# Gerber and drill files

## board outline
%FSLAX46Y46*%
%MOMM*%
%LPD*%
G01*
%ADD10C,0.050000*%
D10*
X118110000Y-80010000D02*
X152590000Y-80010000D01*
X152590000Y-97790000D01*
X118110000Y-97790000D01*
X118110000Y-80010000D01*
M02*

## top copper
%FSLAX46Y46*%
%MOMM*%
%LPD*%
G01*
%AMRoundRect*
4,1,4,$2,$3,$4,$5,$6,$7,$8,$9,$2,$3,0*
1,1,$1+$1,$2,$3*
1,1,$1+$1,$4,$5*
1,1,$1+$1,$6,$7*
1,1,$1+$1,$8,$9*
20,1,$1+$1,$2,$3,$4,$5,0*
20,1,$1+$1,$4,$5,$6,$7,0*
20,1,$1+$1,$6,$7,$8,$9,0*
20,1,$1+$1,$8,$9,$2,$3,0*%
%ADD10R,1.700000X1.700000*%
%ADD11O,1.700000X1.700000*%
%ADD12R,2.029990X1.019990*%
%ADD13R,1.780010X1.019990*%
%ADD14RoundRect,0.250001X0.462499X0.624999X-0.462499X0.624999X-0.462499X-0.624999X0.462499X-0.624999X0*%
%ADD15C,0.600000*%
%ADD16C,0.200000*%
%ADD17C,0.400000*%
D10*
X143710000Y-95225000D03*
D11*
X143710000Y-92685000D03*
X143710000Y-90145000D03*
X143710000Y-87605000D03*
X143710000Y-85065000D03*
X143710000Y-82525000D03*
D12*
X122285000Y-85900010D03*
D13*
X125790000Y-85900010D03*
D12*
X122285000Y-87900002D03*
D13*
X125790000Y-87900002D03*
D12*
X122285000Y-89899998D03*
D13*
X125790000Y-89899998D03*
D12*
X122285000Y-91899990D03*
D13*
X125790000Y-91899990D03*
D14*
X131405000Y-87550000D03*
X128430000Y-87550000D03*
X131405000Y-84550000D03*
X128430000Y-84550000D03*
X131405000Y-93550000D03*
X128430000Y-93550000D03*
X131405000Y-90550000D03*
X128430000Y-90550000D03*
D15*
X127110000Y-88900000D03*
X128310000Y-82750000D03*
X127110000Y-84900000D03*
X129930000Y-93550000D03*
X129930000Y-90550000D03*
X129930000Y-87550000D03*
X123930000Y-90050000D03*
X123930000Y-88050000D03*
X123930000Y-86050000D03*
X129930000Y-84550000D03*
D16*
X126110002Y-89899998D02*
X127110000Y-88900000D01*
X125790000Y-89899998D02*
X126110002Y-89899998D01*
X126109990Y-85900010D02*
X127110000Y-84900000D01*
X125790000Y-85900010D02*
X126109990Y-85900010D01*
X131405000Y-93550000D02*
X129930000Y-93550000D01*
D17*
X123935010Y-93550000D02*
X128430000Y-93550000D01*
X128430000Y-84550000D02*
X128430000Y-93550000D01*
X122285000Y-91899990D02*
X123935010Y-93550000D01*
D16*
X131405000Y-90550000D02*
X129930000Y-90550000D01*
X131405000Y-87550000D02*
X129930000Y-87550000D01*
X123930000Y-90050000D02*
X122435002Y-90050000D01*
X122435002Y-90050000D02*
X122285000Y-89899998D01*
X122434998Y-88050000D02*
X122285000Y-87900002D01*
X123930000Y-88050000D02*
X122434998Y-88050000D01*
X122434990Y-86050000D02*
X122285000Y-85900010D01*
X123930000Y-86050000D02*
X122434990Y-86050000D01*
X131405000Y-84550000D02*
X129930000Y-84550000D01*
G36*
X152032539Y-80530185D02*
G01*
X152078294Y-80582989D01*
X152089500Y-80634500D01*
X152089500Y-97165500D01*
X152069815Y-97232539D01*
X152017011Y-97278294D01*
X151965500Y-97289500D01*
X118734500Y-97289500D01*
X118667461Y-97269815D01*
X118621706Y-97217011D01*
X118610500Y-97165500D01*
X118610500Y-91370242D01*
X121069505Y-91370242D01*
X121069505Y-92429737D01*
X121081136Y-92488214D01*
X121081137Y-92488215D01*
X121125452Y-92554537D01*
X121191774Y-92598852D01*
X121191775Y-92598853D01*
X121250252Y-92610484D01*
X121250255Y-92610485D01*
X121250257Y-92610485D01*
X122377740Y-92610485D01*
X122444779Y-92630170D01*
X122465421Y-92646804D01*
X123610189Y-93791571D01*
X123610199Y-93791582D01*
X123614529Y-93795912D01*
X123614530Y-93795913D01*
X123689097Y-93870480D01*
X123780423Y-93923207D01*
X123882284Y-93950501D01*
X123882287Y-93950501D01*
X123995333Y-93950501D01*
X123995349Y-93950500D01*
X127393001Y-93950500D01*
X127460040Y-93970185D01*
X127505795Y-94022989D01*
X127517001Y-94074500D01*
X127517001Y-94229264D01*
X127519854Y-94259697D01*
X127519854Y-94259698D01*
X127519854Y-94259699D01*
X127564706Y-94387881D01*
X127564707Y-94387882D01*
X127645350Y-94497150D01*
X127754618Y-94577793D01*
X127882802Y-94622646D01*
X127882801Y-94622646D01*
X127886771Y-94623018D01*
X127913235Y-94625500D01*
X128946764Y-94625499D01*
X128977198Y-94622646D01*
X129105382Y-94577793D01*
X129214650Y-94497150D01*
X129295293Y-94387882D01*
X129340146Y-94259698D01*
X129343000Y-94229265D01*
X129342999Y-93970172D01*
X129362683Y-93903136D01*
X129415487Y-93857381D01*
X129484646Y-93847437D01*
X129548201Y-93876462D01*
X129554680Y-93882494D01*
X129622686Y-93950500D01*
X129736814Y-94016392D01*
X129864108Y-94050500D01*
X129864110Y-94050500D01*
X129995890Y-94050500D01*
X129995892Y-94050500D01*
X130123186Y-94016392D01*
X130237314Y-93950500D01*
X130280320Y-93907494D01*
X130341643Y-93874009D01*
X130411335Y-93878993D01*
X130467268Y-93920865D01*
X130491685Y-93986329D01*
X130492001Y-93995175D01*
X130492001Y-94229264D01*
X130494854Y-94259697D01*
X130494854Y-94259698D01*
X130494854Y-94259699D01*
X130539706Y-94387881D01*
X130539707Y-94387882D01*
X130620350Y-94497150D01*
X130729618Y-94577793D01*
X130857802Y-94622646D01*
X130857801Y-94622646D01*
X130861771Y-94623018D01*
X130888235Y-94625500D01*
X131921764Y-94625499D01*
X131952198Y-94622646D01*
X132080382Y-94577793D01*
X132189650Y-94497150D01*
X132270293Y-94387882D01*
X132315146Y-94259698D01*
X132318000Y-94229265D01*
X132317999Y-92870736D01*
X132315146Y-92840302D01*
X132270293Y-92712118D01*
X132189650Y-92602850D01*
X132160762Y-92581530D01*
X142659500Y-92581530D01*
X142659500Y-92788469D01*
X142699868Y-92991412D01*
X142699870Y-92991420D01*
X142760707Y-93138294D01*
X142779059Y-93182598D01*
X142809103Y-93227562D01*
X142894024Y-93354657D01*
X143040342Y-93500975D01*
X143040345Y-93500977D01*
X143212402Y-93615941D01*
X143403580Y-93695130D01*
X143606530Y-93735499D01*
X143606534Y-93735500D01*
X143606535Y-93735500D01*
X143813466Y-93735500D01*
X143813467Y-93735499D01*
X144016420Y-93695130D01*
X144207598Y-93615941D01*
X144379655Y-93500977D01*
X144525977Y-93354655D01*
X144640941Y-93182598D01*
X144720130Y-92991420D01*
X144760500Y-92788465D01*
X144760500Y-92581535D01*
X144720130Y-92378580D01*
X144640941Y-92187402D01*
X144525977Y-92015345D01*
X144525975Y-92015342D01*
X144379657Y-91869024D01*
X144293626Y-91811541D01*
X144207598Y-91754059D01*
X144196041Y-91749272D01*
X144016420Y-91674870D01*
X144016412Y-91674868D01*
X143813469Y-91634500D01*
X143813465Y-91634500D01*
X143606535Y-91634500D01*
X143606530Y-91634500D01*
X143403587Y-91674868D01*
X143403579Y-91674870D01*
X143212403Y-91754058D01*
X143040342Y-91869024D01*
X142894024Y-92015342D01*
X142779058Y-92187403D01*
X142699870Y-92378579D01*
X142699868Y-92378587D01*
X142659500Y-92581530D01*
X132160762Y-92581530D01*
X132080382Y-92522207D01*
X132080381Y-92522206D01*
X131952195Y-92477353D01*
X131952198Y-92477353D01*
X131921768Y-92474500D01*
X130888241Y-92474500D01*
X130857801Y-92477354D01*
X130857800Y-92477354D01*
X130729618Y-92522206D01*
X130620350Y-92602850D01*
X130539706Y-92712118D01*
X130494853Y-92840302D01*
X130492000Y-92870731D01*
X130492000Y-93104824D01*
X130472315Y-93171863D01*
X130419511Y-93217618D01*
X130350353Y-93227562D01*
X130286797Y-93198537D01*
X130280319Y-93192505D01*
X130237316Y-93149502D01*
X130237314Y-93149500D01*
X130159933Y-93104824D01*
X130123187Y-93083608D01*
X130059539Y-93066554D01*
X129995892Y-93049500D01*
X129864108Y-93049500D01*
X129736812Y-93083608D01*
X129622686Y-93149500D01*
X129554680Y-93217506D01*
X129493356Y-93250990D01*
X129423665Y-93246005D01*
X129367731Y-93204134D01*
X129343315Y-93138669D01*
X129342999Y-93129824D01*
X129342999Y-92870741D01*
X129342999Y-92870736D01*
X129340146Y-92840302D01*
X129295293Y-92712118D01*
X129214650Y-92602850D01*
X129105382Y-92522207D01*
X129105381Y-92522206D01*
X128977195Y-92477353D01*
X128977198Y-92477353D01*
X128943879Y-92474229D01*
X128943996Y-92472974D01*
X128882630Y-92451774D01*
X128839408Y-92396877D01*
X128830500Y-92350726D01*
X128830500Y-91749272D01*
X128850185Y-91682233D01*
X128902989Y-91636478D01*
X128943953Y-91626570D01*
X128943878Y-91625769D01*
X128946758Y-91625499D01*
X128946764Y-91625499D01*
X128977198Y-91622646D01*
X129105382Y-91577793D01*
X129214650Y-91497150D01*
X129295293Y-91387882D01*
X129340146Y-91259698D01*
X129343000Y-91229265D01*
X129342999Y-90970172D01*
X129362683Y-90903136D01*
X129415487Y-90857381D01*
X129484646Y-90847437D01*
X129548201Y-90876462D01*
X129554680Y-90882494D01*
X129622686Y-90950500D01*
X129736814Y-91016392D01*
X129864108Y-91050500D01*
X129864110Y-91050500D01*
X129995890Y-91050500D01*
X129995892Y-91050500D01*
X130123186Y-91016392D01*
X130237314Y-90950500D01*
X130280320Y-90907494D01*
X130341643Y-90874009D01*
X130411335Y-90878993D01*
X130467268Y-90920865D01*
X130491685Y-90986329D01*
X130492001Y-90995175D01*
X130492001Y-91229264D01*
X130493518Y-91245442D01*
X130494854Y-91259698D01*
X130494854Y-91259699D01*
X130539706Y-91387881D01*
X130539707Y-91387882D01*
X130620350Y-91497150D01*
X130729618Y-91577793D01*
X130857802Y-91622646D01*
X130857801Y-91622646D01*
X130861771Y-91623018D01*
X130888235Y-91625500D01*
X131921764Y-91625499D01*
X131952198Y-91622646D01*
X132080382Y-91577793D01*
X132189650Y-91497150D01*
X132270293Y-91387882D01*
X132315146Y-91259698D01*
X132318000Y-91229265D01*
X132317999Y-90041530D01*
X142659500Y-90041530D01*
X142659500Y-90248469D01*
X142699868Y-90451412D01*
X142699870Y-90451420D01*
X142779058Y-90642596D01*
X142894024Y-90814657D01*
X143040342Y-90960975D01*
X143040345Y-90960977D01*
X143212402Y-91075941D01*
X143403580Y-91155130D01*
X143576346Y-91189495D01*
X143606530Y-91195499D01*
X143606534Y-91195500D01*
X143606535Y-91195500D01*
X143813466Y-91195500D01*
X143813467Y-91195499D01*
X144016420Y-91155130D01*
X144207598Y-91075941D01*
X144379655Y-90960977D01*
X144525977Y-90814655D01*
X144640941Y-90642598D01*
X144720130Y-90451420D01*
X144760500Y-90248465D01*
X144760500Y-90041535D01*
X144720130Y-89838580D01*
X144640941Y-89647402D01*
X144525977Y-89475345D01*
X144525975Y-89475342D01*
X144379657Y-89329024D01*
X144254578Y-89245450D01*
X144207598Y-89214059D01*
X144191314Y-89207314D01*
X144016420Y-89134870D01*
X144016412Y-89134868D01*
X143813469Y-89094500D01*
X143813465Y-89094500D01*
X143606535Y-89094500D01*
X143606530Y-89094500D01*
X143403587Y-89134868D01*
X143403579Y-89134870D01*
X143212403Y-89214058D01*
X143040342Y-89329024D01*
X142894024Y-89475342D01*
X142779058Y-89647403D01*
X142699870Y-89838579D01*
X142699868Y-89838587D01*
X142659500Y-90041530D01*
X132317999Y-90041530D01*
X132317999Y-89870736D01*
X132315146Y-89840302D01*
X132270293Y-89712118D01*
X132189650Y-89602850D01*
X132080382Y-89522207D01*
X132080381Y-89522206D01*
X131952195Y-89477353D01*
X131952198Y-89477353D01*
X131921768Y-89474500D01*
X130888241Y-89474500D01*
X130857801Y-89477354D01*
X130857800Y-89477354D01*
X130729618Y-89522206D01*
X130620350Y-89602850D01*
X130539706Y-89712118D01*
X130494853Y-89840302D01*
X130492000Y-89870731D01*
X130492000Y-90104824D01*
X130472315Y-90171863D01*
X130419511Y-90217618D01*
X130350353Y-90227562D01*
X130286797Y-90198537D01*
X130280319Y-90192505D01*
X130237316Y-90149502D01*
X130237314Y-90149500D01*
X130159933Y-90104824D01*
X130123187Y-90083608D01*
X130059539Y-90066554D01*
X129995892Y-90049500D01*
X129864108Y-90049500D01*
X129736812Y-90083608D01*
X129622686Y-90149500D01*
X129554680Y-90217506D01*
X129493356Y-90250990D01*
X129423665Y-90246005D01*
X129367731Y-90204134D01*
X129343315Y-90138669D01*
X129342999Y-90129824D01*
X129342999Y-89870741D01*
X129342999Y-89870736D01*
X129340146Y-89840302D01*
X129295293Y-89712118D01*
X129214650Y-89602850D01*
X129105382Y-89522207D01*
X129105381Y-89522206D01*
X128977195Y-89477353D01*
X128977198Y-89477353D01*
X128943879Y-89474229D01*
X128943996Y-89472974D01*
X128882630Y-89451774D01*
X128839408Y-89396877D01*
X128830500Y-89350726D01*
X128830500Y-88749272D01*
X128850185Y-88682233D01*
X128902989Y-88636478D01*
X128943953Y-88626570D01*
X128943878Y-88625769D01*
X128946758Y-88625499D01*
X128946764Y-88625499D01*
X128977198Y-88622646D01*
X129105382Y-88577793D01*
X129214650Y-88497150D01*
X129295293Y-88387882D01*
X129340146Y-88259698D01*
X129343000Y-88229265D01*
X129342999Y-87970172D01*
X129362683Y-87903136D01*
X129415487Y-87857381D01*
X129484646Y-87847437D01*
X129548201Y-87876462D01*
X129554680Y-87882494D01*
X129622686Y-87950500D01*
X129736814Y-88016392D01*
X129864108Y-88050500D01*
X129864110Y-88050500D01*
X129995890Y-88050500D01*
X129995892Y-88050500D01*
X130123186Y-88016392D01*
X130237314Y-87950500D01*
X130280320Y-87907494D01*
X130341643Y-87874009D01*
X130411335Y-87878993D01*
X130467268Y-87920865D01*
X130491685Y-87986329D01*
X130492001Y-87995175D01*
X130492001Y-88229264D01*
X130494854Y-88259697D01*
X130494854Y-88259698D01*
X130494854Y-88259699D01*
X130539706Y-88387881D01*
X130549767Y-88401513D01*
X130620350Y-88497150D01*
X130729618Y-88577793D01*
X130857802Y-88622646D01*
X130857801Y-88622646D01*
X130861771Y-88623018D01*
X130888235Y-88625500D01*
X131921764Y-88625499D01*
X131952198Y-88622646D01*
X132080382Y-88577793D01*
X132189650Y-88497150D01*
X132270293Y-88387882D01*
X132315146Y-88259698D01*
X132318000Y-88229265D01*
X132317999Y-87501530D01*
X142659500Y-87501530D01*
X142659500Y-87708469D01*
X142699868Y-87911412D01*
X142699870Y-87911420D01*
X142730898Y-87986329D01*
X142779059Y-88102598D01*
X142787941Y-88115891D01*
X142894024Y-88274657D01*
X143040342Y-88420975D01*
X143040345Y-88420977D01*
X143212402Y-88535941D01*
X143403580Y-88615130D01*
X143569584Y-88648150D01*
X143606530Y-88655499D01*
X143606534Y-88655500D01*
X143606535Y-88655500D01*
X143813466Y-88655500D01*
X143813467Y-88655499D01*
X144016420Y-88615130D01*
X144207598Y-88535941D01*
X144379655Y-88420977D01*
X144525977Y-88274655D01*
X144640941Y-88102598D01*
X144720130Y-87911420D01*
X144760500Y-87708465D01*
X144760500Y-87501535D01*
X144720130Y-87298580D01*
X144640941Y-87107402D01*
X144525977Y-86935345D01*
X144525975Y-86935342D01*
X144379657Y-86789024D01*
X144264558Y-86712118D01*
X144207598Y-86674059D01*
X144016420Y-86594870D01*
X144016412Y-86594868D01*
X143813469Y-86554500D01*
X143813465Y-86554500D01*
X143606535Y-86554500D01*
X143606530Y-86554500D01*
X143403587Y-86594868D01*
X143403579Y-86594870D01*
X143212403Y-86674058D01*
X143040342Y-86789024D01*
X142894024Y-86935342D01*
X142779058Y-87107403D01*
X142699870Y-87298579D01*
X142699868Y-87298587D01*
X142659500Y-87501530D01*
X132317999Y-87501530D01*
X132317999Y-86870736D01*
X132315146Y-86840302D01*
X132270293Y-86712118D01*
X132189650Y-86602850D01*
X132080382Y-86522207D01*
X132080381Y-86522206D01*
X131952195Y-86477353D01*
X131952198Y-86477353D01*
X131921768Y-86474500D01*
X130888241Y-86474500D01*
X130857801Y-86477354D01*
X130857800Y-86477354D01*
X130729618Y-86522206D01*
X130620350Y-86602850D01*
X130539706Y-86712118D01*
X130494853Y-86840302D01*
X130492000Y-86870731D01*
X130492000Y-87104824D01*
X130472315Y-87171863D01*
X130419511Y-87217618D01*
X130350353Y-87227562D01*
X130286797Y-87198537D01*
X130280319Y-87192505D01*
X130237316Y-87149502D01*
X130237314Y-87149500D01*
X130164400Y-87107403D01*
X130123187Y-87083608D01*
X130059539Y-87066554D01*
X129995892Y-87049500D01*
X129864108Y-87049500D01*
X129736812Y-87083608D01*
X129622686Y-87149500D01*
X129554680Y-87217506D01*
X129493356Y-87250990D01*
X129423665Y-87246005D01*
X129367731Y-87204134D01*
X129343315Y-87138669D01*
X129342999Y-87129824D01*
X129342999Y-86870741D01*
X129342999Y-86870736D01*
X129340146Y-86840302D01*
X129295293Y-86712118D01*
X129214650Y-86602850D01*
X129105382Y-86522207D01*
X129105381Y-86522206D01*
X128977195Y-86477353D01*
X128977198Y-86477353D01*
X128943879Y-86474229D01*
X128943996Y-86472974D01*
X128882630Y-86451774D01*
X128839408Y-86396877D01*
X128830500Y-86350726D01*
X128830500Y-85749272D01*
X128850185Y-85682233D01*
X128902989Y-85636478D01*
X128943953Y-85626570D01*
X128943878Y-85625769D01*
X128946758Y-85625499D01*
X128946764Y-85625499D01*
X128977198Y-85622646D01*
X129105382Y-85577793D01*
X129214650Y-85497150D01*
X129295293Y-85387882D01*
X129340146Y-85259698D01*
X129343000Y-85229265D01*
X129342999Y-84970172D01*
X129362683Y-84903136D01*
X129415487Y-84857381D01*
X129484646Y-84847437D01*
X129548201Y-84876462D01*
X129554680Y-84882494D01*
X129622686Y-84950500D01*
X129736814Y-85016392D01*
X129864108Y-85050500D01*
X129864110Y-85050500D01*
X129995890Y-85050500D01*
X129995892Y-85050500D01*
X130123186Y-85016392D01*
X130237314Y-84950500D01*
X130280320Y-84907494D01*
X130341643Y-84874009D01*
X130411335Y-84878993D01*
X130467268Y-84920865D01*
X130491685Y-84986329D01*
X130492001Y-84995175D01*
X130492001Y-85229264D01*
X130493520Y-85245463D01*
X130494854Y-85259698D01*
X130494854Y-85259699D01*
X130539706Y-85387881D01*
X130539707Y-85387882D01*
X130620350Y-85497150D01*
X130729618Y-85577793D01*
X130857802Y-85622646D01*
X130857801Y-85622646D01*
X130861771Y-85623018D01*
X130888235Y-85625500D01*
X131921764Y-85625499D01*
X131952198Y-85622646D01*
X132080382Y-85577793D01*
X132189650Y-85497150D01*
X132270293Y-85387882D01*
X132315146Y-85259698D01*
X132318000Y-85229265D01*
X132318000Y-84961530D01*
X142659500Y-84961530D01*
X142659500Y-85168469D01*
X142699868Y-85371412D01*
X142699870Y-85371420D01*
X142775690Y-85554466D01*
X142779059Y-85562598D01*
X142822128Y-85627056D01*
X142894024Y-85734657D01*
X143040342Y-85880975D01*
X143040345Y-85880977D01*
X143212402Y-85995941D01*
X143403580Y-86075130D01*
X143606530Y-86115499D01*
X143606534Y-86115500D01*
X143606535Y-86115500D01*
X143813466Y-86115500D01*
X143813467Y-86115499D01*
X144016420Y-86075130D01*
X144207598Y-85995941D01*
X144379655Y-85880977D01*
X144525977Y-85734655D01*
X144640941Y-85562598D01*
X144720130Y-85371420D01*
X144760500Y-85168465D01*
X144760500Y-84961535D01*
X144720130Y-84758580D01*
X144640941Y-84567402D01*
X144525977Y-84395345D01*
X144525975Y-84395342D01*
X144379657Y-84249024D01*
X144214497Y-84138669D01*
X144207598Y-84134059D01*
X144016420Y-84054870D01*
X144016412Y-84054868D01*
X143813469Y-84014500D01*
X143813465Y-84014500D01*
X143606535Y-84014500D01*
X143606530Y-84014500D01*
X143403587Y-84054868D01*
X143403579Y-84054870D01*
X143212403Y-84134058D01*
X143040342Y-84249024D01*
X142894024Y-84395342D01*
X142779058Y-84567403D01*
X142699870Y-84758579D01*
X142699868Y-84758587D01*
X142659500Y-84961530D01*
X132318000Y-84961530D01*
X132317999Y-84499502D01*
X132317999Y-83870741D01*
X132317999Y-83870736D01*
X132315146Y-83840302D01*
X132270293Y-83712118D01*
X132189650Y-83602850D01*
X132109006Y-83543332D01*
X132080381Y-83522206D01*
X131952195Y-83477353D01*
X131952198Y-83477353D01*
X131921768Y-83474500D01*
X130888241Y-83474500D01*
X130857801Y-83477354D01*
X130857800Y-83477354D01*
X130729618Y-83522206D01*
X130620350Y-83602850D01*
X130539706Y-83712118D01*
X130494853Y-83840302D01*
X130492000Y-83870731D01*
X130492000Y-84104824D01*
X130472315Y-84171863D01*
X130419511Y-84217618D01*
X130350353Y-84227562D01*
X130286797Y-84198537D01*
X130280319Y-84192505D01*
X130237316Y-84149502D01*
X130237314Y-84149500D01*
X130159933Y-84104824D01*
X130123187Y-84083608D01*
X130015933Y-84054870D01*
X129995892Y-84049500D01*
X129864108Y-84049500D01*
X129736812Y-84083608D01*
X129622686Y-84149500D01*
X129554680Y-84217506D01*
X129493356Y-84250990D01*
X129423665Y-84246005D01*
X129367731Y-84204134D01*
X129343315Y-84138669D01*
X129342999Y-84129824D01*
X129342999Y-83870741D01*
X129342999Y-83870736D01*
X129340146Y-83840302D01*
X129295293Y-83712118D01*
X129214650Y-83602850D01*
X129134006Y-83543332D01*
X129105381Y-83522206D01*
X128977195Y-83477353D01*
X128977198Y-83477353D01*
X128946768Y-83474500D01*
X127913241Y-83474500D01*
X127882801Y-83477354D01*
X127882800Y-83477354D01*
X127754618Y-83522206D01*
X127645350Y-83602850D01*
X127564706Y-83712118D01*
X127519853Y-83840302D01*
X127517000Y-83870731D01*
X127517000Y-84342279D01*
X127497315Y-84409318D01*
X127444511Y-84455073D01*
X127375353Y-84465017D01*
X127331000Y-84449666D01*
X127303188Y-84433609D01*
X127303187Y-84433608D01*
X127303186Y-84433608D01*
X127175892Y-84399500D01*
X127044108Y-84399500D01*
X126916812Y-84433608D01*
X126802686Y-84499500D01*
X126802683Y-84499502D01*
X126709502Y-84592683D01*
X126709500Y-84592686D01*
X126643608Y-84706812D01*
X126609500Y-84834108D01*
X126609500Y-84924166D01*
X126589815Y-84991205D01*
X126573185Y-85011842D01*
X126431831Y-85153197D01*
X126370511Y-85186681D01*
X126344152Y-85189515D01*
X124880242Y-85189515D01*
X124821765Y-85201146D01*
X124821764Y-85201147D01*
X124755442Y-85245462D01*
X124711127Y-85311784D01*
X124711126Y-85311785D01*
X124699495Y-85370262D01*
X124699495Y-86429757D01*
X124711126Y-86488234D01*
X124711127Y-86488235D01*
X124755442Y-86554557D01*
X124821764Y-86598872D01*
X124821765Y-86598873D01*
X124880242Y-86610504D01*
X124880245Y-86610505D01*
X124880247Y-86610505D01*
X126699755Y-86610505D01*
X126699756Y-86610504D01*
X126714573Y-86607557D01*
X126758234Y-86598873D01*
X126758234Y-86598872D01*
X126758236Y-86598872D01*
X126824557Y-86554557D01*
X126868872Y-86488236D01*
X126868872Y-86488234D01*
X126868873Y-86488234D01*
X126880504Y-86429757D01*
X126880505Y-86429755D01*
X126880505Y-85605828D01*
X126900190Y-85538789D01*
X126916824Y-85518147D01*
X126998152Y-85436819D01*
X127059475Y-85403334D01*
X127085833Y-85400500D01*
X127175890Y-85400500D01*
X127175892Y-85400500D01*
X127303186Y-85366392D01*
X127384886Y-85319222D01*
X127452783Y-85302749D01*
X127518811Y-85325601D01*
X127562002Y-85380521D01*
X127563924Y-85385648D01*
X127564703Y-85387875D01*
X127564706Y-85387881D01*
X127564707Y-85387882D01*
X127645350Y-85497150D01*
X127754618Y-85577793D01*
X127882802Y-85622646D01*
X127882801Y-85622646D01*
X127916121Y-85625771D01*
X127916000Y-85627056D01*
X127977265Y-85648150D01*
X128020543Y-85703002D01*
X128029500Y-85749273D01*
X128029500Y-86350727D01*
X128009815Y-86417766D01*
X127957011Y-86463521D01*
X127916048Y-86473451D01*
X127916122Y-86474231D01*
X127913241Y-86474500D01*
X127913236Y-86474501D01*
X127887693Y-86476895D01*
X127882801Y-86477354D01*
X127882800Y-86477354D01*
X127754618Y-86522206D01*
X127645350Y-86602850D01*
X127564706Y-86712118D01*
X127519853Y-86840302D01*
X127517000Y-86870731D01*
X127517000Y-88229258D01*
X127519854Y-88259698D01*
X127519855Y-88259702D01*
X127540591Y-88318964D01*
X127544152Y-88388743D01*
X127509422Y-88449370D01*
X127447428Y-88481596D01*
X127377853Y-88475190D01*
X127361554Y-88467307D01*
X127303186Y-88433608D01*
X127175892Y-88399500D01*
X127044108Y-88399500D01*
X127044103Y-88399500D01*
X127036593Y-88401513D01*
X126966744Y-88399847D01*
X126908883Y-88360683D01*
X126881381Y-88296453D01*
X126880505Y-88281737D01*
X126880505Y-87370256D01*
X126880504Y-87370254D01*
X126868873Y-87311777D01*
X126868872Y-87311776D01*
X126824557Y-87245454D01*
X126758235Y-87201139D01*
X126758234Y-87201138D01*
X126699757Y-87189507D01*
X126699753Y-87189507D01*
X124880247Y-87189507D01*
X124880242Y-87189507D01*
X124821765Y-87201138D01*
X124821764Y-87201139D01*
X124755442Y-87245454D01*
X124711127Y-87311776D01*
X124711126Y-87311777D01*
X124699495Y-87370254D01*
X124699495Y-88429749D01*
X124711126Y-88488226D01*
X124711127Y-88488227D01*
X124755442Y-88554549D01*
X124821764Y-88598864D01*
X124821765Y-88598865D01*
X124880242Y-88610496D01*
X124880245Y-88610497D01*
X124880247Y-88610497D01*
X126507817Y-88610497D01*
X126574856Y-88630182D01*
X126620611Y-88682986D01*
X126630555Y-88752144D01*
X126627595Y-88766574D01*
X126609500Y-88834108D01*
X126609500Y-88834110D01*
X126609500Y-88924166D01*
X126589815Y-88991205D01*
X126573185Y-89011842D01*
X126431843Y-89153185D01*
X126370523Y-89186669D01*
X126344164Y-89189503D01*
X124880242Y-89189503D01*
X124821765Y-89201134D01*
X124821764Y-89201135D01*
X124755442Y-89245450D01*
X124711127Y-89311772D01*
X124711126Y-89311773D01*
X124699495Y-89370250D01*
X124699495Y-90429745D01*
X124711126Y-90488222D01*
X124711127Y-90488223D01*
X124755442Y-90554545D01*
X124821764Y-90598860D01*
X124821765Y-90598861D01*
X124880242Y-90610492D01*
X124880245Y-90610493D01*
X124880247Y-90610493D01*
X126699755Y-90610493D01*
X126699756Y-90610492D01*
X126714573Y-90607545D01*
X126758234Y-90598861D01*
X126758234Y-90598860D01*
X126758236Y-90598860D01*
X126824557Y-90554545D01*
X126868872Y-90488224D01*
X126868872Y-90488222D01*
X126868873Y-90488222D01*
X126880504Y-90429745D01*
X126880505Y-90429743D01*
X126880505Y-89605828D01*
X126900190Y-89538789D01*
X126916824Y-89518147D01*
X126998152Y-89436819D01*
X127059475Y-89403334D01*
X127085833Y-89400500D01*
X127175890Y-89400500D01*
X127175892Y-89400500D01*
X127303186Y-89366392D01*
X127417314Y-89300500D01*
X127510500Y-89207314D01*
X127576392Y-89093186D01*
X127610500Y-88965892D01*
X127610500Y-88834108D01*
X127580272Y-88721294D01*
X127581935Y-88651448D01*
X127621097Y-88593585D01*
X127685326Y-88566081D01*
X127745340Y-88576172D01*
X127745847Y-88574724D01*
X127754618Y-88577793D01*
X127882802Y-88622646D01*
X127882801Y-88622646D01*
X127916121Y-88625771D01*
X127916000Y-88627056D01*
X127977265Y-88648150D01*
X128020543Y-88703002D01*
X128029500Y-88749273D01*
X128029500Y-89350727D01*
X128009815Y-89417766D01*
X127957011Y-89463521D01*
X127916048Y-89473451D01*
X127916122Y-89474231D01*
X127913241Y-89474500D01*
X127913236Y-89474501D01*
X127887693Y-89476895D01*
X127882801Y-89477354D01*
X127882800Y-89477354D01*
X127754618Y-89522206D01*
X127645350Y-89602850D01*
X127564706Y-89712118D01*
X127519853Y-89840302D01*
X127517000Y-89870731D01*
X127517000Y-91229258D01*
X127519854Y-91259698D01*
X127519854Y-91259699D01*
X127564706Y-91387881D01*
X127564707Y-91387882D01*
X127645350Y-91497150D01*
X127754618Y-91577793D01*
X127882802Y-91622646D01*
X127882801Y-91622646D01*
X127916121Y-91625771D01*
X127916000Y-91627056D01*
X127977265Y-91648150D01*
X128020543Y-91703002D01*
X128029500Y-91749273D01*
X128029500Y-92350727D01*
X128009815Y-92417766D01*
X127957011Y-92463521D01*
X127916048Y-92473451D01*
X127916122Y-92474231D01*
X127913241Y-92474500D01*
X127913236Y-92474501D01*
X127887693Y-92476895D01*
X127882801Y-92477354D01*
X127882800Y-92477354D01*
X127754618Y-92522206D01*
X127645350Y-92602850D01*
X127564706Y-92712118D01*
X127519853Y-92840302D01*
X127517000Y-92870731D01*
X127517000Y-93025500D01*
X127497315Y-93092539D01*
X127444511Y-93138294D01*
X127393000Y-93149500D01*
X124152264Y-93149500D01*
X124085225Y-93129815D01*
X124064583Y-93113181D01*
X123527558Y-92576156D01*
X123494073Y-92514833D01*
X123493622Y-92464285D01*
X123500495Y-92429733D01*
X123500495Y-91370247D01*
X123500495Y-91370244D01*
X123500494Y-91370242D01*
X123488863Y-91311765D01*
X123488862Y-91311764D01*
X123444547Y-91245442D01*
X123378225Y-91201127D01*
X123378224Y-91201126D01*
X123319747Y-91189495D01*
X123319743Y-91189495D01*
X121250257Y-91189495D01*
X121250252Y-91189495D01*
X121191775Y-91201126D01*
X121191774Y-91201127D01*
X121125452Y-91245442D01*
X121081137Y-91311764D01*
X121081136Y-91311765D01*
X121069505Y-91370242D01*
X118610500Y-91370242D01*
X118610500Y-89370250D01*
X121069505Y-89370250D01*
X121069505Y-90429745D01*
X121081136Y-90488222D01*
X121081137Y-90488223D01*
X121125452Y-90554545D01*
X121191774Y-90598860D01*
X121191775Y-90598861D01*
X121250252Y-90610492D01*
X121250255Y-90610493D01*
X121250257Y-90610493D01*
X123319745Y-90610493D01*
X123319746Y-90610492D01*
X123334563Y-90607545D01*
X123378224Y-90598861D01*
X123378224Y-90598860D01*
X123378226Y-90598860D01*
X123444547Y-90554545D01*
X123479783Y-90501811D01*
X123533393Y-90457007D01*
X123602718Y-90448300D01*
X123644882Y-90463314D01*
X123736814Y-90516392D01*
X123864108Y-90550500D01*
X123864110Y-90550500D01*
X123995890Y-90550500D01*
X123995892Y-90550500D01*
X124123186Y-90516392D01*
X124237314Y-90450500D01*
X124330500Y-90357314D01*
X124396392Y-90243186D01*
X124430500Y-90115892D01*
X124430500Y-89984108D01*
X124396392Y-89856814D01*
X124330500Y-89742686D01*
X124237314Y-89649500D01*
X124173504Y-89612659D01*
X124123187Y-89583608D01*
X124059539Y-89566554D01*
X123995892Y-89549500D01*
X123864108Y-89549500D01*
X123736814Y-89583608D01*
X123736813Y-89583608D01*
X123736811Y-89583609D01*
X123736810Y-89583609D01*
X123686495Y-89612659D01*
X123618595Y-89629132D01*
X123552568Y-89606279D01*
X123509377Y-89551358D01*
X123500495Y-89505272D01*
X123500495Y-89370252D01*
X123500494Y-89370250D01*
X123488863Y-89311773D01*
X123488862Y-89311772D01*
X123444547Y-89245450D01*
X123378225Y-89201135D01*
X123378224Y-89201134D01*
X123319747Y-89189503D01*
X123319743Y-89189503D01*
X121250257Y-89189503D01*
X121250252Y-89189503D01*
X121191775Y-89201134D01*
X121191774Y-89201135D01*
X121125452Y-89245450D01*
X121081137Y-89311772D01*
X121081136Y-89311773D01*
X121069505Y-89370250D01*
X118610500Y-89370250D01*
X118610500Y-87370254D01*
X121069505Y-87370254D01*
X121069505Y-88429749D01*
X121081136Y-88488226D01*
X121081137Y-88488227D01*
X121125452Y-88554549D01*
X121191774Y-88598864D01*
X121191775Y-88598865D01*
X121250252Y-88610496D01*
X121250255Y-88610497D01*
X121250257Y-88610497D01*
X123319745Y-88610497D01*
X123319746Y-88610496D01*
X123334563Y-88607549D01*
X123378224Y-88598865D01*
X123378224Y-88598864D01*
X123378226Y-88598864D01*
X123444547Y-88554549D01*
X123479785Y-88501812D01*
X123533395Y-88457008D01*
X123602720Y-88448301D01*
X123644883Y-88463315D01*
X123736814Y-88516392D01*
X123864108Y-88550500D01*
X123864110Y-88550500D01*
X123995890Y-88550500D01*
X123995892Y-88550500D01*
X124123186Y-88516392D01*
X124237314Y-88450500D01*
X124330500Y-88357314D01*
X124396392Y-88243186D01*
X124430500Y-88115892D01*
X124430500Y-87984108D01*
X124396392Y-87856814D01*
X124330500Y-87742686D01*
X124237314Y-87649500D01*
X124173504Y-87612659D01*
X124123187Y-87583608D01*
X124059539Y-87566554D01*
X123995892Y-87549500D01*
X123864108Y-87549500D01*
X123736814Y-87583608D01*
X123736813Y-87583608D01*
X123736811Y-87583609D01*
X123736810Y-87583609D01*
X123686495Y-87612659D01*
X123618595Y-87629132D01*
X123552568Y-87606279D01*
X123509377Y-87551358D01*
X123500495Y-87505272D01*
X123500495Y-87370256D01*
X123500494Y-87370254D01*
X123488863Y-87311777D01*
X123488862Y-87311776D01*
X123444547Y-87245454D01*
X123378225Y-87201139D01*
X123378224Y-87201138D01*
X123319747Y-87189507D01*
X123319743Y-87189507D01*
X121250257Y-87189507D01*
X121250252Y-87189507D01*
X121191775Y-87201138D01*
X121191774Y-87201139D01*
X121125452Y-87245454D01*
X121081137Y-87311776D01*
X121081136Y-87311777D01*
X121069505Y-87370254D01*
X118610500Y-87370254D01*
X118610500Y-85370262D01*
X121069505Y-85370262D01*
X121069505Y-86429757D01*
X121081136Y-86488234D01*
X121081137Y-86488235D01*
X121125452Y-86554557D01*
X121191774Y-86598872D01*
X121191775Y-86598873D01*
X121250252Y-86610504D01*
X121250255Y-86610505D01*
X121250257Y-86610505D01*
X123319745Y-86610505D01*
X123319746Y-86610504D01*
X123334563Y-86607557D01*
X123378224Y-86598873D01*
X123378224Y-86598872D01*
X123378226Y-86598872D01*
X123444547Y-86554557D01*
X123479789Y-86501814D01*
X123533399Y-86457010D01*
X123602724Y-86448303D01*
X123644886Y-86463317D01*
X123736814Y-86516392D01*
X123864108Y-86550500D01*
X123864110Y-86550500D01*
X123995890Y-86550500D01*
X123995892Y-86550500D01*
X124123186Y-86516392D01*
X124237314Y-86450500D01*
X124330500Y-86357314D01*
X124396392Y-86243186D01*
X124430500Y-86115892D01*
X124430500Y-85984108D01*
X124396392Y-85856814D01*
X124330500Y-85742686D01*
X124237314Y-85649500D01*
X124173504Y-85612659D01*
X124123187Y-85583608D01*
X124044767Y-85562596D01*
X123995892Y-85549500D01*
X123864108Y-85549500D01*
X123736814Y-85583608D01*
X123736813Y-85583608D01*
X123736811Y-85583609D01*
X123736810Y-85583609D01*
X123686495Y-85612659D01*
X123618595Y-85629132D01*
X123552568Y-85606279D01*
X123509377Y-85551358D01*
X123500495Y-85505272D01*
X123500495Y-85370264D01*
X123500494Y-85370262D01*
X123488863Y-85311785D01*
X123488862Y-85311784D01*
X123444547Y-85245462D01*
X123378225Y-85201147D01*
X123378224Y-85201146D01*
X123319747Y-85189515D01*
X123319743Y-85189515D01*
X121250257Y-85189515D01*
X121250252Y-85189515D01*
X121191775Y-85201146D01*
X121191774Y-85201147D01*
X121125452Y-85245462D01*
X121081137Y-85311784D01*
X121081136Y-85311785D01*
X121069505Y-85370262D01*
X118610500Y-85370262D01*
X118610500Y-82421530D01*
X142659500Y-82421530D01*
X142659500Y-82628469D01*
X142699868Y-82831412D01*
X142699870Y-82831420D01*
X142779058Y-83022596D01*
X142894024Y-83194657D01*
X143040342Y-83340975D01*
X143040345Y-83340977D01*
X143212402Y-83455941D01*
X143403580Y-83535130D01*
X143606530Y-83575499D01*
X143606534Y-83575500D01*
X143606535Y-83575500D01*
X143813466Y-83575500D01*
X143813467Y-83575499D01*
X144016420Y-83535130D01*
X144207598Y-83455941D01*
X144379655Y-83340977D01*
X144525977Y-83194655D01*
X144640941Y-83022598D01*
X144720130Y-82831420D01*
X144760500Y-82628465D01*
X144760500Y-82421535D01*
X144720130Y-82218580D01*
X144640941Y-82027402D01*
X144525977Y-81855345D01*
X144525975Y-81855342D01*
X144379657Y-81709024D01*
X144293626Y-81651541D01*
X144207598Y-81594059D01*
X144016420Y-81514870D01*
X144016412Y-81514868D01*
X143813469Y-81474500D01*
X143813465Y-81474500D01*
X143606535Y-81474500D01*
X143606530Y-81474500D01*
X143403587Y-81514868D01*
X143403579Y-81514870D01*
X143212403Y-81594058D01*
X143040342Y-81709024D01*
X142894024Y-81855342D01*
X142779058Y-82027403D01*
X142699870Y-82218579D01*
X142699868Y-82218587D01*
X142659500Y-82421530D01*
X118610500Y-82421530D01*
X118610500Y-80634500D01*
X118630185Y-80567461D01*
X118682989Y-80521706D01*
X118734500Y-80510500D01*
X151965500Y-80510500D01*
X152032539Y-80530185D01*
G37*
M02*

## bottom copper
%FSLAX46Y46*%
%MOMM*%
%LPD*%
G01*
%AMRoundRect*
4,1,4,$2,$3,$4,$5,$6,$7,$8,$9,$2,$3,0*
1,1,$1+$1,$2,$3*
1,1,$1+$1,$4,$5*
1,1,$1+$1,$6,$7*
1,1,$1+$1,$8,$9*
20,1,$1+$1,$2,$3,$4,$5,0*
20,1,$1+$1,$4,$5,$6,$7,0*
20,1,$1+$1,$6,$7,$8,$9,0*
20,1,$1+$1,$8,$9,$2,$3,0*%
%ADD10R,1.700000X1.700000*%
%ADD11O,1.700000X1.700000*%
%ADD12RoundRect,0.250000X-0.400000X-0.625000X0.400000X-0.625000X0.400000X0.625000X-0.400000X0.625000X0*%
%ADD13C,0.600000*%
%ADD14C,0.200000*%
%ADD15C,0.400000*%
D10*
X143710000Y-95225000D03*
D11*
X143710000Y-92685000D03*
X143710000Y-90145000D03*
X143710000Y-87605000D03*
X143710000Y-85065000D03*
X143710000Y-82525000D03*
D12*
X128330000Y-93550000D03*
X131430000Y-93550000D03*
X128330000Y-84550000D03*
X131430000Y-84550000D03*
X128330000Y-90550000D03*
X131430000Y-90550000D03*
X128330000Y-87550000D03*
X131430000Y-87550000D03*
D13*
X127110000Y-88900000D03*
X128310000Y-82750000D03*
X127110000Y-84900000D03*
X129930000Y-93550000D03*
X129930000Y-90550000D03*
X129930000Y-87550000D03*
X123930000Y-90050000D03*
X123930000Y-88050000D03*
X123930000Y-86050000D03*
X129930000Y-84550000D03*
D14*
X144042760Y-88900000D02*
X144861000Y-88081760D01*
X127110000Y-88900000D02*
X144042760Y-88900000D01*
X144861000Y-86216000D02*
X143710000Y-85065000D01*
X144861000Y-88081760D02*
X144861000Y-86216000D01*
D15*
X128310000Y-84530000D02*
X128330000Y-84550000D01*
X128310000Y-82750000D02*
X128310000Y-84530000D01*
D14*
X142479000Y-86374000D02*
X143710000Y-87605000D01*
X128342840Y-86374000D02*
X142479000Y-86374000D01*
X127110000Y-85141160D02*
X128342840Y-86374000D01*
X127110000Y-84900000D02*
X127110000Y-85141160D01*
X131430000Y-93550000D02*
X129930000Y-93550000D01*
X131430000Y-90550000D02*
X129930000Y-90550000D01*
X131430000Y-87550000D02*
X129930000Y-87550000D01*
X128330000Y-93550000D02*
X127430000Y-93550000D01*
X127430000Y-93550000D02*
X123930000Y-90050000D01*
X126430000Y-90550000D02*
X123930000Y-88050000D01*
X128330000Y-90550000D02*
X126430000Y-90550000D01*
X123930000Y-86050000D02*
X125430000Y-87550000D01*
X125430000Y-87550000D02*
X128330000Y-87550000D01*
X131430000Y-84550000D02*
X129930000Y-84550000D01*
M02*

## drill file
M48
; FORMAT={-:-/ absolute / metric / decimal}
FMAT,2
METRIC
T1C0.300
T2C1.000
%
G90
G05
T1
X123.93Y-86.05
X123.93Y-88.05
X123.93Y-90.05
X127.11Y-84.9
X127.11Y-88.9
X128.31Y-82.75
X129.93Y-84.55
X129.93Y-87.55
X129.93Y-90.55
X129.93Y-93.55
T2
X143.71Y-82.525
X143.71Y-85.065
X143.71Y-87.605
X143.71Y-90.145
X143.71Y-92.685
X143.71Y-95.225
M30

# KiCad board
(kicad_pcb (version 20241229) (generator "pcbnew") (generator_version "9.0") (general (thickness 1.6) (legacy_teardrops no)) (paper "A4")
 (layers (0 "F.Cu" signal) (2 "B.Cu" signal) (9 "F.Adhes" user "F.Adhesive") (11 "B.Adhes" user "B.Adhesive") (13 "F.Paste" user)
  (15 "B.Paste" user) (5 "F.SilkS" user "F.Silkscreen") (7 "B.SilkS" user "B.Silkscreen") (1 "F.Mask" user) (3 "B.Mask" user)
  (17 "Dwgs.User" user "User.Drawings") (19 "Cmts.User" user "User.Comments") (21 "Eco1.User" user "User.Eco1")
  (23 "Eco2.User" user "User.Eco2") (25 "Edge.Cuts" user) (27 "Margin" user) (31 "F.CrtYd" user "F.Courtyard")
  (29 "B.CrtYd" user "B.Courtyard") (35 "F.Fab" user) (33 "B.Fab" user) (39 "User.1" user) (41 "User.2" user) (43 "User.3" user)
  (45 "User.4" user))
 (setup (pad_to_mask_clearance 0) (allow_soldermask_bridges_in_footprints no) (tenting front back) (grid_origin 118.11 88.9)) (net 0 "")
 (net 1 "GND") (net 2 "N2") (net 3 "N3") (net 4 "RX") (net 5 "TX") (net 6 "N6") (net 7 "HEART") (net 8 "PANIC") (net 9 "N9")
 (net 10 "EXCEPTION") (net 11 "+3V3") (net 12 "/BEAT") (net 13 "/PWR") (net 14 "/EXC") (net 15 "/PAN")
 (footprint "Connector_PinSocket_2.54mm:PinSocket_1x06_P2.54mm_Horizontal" (layer "F.Cu") (at 143.71 95.225 180)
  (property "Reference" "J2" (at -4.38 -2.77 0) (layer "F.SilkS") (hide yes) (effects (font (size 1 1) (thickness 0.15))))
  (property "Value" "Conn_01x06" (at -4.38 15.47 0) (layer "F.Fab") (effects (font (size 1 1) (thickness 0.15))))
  (pad "1" thru_hole rect (at 0 0 180) (size 1.7 1.7) (drill 1) (layers "*.Cu" "*.Mask") (remove_unused_layers no) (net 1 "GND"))
  (pad "2" thru_hole oval (at 0 2.54 180) (size 1.7 1.7) (drill 1) (layers "*.Cu" "*.Mask") (remove_unused_layers no) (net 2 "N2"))
  (pad "3" thru_hole oval (at 0 5.08 180) (size 1.7 1.7) (drill 1) (layers "*.Cu" "*.Mask") (remove_unused_layers no) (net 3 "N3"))
  (pad "4" thru_hole oval (at 0 7.62 180) (size 1.7 1.7) (drill 1) (layers "*.Cu" "*.Mask") (remove_unused_layers no) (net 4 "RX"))
  (pad "5" thru_hole oval (at 0 10.16 180) (size 1.7 1.7) (drill 1) (layers "*.Cu" "*.Mask") (remove_unused_layers no) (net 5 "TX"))
  (pad "6" thru_hole oval (at 0 12.7 180) (size 1.7 1.7) (drill 1) (layers "*.Cu" "*.Mask") (remove_unused_layers no) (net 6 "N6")))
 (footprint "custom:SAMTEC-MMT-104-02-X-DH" (layer "F.Cu") (at 119.11 88.9 -90)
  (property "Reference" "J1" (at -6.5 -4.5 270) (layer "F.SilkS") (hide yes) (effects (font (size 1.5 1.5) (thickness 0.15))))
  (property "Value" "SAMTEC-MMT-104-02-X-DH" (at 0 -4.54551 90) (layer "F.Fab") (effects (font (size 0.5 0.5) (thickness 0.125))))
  (pad "1" smd rect (at -2.99999 -3.175 270) (size 1.01999 2.02999) (layers "F.Cu" "F.Paste") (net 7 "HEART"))
  (pad "2" smd rect (at -2.99999 -6.68 270) (size 1.01999 1.78001) (layers "F.Cu" "F.Paste") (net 4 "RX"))
  (pad "3" smd rect (at -0.999998 -3.175 270) (size 1.01999 2.02999) (layers "F.Cu" "F.Paste") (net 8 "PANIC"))
  (pad "4" smd rect (at -0.999998 -6.68 270) (size 1.01999 1.78001) (layers "F.Cu" "F.Paste") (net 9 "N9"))
  (pad "5" smd rect (at 0.999998 -3.175 270) (size 1.01999 2.02999) (layers "F.Cu" "F.Paste") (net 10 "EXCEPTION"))
  (pad "6" smd rect (at 0.999998 -6.68 270) (size 1.01999 1.78001) (layers "F.Cu" "F.Paste") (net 5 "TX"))
  (pad "7" smd rect (at 2.99999 -3.175 270) (size 1.01999 2.02999) (layers "F.Cu" "F.Paste") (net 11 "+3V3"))
  (pad "8" smd rect (at 2.99999 -6.68 270) (size 1.01999 1.78001) (layers "F.Cu" "F.Paste") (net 1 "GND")))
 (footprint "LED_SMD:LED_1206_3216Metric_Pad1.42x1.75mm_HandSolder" (layer "F.Cu") (at 129.9175 87.55 180)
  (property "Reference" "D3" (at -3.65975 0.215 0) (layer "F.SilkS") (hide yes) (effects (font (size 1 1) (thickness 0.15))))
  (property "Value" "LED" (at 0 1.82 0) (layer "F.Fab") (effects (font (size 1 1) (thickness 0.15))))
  (pad "1" smd roundrect (at -1.4875 0 180) (size 1.425 1.75) (layers "F.Cu" "F.Mask" "F.Paste") (roundrect_rratio 0.175439)
   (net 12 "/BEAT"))
  (pad "2" smd roundrect (at 1.4875 0 180) (size 1.425 1.75) (layers "F.Cu" "F.Mask" "F.Paste") (roundrect_rratio 0.175439) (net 11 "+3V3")))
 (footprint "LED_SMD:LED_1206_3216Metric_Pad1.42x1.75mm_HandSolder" (layer "F.Cu") (at 129.9175 84.55 180)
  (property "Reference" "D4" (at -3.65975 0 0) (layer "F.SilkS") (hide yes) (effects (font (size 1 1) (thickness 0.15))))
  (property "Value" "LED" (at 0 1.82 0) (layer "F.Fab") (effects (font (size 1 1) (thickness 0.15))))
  (pad "1" smd roundrect (at -1.4875 0 180) (size 1.425 1.75) (layers "F.Cu" "F.Mask" "F.Paste") (roundrect_rratio 0.175439) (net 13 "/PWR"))
  (pad "2" smd roundrect (at 1.4875 0 180) (size 1.425 1.75) (layers "F.Cu" "F.Mask" "F.Paste") (roundrect_rratio 0.175439) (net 11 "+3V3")))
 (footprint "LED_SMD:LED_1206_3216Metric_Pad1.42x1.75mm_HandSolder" (layer "F.Cu") (at 129.9175 93.55 180)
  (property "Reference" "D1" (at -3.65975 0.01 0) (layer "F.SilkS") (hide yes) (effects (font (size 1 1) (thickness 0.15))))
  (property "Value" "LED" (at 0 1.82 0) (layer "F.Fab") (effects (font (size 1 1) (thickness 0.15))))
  (pad "1" smd roundrect (at -1.4875 0 180) (size 1.425 1.75) (layers "F.Cu" "F.Mask" "F.Paste") (roundrect_rratio 0.175439) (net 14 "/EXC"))
  (pad "2" smd roundrect (at 1.4875 0 180) (size 1.425 1.75) (layers "F.Cu" "F.Mask" "F.Paste") (roundrect_rratio 0.175439) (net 11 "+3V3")))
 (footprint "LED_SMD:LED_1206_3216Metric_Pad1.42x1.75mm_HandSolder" (layer "F.Cu") (at 129.9175 90.55 180)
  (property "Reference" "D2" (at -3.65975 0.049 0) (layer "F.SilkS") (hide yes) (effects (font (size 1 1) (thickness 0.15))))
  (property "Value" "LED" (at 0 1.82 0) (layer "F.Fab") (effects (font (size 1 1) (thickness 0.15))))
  (pad "1" smd roundrect (at -1.4875 0 180) (size 1.425 1.75) (layers "F.Cu" "F.Mask" "F.Paste") (roundrect_rratio 0.175439) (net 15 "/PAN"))
  (pad "2" smd roundrect (at 1.4875 0 180) (size 1.425 1.75) (layers "F.Cu" "F.Mask" "F.Paste") (roundrect_rratio 0.175439) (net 11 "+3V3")))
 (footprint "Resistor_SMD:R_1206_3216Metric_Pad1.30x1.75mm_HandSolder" (layer "B.Cu") (at 129.88 93.55)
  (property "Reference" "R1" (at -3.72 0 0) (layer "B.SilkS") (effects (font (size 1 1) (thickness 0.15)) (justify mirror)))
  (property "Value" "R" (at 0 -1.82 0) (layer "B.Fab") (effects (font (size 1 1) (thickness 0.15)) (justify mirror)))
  (pad "1" smd roundrect (at -1.55 0) (size 1.3 1.75) (layers "B.Cu" "B.Mask" "B.Paste") (roundrect_rratio 0.192308) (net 10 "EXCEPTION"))
  (pad "2" smd roundrect (at 1.55 0) (size 1.3 1.75) (layers "B.Cu" "B.Mask" "B.Paste") (roundrect_rratio 0.192308) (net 14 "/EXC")))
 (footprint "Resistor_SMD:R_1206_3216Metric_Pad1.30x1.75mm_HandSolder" (layer "B.Cu") (at 129.88 84.55)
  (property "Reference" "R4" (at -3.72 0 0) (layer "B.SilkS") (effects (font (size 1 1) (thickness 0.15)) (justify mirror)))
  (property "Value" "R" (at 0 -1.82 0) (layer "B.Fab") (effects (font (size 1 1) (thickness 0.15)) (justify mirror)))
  (pad "1" smd roundrect (at -1.55 0) (size 1.3 1.75) (layers "B.Cu" "B.Mask" "B.Paste") (roundrect_rratio 0.192308) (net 1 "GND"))
  (pad "2" smd roundrect (at 1.55 0) (size 1.3 1.75) (layers "B.Cu" "B.Mask" "B.Paste") (roundrect_rratio 0.192308) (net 13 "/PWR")))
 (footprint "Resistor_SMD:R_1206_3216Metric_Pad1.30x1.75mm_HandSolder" (layer "B.Cu") (at 129.88 90.55)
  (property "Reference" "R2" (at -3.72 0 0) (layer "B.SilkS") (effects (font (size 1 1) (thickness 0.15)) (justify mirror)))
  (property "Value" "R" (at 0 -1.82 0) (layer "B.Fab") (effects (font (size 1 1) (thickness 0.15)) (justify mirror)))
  (pad "1" smd roundrect (at -1.55 0) (size 1.3 1.75) (layers "B.Cu" "B.Mask" "B.Paste") (roundrect_rratio 0.192308) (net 8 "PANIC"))
  (pad "2" smd roundrect (at 1.55 0) (size 1.3 1.75) (layers "B.Cu" "B.Mask" "B.Paste") (roundrect_rratio 0.192308) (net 15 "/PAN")))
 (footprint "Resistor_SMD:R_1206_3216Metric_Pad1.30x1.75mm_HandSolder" (layer "B.Cu") (at 129.88 87.55)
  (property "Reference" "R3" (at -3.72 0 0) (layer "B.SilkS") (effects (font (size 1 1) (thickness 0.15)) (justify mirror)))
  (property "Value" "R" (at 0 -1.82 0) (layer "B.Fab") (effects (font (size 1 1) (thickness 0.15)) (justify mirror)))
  (pad "1" smd roundrect (at -1.55 0) (size 1.3 1.75) (layers "B.Cu" "B.Mask" "B.Paste") (roundrect_rratio 0.192308) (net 7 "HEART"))
  (pad "2" smd roundrect (at 1.55 0) (size 1.3 1.75) (layers "B.Cu" "B.Mask" "B.Paste") (roundrect_rratio 0.192308) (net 12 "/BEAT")))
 (gr_rect (start 118.11 80.01) (end 152.59 97.79) (stroke (width 0.05) (type default)) (fill no) (layer "Edge.Cuts"))
 (segment (start 126.110002 89.899998) (end 127.11 88.9) (width 0.2) (layer "F.Cu") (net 5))
 (segment (start 125.79 89.899998) (end 126.110002 89.899998) (width 0.2) (layer "F.Cu") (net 5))
 (via (at 127.11 88.9) (size 0.6) (drill 0.3) (layers "F.Cu" "B.Cu") (free yes) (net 5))
 (segment (start 144.04276 88.9) (end 144.861 88.08176) (width 0.2) (layer "B.Cu") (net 5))
 (segment (start 127.11 88.9) (end 144.04276 88.9) (width 0.2) (layer "B.Cu") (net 5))
 (segment (start 144.861 86.216) (end 143.71 85.065) (width 0.2) (layer "B.Cu") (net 5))
 (segment (start 144.861 88.08176) (end 144.861 86.216) (width 0.2) (layer "B.Cu") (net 5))
 (via (at 128.31 82.75) (size 0.6) (drill 0.3) (layers "F.Cu" "B.Cu") (free yes) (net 1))
 (segment (start 128.31 84.53) (end 128.33 84.55) (width 0.4) (layer "B.Cu") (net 1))
 (segment (start 128.31 82.75) (end 128.31 84.53) (width 0.4) (layer "B.Cu") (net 1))
 (segment (start 126.10999 85.90001) (end 127.11 84.9) (width 0.2) (layer "F.Cu") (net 4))
 (segment (start 125.79 85.90001) (end 126.10999 85.90001) (width 0.2) (layer "F.Cu") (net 4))
 (via (at 127.11 84.9) (size 0.6) (drill 0.3) (layers "F.Cu" "B.Cu") (free yes) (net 4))
 (segment (start 142.479 86.374) (end 143.71 87.605) (width 0.2) (layer "B.Cu") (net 4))
 (segment (start 128.34284 86.374) (end 142.479 86.374) (width 0.2) (layer "B.Cu") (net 4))
 (segment (start 127.11 85.14116) (end 128.34284 86.374) (width 0.2) (layer "B.Cu") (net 4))
 (segment (start 127.11 84.9) (end 127.11 85.14116) (width 0.2) (layer "B.Cu") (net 4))
 (segment (start 131.405 93.55) (end 129.93 93.55) (width 0.2) (layer "F.Cu") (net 14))
 (via (at 129.93 93.55) (size 0.6) (drill 0.3) (layers "F.Cu" "B.Cu") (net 14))
 (segment (start 131.43 93.55) (end 129.93 93.55) (width 0.2) (layer "B.Cu") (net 14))
 (segment (start 123.93501 93.55) (end 128.43 93.55) (width 0.4) (layer "F.Cu") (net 11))
 (segment (start 128.43 84.55) (end 128.43 93.55) (width 0.4) (layer "F.Cu") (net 11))
 (segment (start 122.285 91.89999) (end 123.93501 93.55) (width 0.4) (layer "F.Cu") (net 11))
 (segment (start 131.405 90.55) (end 129.93 90.55) (width 0.2) (layer "F.Cu") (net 15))
 (via (at 129.93 90.55) (size 0.6) (drill 0.3) (layers "F.Cu" "B.Cu") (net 15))
 (segment (start 131.43 90.55) (end 129.93 90.55) (width 0.2) (layer "B.Cu") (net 15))
 (segment (start 131.405 87.55) (end 129.93 87.55) (width 0.2) (layer "F.Cu") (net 12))
 (via (at 129.93 87.55) (size 0.6) (drill 0.3) (layers "F.Cu" "B.Cu") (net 12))
 (segment (start 131.43 87.55) (end 129.93 87.55) (width 0.2) (layer "B.Cu") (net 12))
 (segment (start 123.93 90.05) (end 122.435002 90.05) (width 0.2) (layer "F.Cu") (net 10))
 (segment (start 122.435002 90.05) (end 122.285 89.899998) (width 0.2) (layer "F.Cu") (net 10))
 (via (at 123.93 90.05) (size 0.6) (drill 0.3) (layers "F.Cu" "B.Cu") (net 10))
 (segment (start 128.33 93.55) (end 127.43 93.55) (width 0.2) (layer "B.Cu") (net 10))
 (segment (start 127.43 93.55) (end 123.93 90.05) (width 0.2) (layer "B.Cu") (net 10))
 (segment (start 122.434998 88.05) (end 122.285 87.900002) (width 0.2) (layer "F.Cu") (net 8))
 (segment (start 123.93 88.05) (end 122.434998 88.05) (width 0.2) (layer "F.Cu") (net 8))
 (via (at 123.93 88.05) (size 0.6) (drill 0.3) (layers "F.Cu" "B.Cu") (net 8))
 (segment (start 126.43 90.55) (end 123.93 88.05) (width 0.2) (layer "B.Cu") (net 8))
 (segment (start 128.33 90.55) (end 126.43 90.55) (width 0.2) (layer "B.Cu") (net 8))
 (segment (start 122.43499 86.05) (end 122.285 85.90001) (width 0.2) (layer "F.Cu") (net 7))
 (segment (start 123.93 86.05) (end 122.43499 86.05) (width 0.2) (layer "F.Cu") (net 7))
 (via (at 123.93 86.05) (size 0.6) (drill 0.3) (layers "F.Cu" "B.Cu") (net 7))
 (segment (start 123.93 86.05) (end 125.43 87.55) (width 0.2) (layer "B.Cu") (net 7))
 (segment (start 125.43 87.55) (end 128.33 87.55) (width 0.2) (layer "B.Cu") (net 7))
 (segment (start 131.405 84.55) (end 129.93 84.55) (width 0.2) (layer "F.Cu") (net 13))
 (via (at 129.93 84.55) (size 0.6) (drill 0.3) (layers "F.Cu" "B.Cu") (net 13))
 (segment (start 131.43 84.55) (end 129.93 84.55) (width 0.2) (layer "B.Cu") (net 13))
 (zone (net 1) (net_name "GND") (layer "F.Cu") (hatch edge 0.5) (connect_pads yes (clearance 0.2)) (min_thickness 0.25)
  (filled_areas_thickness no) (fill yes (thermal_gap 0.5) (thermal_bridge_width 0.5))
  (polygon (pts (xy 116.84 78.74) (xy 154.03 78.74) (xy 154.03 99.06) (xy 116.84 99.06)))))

